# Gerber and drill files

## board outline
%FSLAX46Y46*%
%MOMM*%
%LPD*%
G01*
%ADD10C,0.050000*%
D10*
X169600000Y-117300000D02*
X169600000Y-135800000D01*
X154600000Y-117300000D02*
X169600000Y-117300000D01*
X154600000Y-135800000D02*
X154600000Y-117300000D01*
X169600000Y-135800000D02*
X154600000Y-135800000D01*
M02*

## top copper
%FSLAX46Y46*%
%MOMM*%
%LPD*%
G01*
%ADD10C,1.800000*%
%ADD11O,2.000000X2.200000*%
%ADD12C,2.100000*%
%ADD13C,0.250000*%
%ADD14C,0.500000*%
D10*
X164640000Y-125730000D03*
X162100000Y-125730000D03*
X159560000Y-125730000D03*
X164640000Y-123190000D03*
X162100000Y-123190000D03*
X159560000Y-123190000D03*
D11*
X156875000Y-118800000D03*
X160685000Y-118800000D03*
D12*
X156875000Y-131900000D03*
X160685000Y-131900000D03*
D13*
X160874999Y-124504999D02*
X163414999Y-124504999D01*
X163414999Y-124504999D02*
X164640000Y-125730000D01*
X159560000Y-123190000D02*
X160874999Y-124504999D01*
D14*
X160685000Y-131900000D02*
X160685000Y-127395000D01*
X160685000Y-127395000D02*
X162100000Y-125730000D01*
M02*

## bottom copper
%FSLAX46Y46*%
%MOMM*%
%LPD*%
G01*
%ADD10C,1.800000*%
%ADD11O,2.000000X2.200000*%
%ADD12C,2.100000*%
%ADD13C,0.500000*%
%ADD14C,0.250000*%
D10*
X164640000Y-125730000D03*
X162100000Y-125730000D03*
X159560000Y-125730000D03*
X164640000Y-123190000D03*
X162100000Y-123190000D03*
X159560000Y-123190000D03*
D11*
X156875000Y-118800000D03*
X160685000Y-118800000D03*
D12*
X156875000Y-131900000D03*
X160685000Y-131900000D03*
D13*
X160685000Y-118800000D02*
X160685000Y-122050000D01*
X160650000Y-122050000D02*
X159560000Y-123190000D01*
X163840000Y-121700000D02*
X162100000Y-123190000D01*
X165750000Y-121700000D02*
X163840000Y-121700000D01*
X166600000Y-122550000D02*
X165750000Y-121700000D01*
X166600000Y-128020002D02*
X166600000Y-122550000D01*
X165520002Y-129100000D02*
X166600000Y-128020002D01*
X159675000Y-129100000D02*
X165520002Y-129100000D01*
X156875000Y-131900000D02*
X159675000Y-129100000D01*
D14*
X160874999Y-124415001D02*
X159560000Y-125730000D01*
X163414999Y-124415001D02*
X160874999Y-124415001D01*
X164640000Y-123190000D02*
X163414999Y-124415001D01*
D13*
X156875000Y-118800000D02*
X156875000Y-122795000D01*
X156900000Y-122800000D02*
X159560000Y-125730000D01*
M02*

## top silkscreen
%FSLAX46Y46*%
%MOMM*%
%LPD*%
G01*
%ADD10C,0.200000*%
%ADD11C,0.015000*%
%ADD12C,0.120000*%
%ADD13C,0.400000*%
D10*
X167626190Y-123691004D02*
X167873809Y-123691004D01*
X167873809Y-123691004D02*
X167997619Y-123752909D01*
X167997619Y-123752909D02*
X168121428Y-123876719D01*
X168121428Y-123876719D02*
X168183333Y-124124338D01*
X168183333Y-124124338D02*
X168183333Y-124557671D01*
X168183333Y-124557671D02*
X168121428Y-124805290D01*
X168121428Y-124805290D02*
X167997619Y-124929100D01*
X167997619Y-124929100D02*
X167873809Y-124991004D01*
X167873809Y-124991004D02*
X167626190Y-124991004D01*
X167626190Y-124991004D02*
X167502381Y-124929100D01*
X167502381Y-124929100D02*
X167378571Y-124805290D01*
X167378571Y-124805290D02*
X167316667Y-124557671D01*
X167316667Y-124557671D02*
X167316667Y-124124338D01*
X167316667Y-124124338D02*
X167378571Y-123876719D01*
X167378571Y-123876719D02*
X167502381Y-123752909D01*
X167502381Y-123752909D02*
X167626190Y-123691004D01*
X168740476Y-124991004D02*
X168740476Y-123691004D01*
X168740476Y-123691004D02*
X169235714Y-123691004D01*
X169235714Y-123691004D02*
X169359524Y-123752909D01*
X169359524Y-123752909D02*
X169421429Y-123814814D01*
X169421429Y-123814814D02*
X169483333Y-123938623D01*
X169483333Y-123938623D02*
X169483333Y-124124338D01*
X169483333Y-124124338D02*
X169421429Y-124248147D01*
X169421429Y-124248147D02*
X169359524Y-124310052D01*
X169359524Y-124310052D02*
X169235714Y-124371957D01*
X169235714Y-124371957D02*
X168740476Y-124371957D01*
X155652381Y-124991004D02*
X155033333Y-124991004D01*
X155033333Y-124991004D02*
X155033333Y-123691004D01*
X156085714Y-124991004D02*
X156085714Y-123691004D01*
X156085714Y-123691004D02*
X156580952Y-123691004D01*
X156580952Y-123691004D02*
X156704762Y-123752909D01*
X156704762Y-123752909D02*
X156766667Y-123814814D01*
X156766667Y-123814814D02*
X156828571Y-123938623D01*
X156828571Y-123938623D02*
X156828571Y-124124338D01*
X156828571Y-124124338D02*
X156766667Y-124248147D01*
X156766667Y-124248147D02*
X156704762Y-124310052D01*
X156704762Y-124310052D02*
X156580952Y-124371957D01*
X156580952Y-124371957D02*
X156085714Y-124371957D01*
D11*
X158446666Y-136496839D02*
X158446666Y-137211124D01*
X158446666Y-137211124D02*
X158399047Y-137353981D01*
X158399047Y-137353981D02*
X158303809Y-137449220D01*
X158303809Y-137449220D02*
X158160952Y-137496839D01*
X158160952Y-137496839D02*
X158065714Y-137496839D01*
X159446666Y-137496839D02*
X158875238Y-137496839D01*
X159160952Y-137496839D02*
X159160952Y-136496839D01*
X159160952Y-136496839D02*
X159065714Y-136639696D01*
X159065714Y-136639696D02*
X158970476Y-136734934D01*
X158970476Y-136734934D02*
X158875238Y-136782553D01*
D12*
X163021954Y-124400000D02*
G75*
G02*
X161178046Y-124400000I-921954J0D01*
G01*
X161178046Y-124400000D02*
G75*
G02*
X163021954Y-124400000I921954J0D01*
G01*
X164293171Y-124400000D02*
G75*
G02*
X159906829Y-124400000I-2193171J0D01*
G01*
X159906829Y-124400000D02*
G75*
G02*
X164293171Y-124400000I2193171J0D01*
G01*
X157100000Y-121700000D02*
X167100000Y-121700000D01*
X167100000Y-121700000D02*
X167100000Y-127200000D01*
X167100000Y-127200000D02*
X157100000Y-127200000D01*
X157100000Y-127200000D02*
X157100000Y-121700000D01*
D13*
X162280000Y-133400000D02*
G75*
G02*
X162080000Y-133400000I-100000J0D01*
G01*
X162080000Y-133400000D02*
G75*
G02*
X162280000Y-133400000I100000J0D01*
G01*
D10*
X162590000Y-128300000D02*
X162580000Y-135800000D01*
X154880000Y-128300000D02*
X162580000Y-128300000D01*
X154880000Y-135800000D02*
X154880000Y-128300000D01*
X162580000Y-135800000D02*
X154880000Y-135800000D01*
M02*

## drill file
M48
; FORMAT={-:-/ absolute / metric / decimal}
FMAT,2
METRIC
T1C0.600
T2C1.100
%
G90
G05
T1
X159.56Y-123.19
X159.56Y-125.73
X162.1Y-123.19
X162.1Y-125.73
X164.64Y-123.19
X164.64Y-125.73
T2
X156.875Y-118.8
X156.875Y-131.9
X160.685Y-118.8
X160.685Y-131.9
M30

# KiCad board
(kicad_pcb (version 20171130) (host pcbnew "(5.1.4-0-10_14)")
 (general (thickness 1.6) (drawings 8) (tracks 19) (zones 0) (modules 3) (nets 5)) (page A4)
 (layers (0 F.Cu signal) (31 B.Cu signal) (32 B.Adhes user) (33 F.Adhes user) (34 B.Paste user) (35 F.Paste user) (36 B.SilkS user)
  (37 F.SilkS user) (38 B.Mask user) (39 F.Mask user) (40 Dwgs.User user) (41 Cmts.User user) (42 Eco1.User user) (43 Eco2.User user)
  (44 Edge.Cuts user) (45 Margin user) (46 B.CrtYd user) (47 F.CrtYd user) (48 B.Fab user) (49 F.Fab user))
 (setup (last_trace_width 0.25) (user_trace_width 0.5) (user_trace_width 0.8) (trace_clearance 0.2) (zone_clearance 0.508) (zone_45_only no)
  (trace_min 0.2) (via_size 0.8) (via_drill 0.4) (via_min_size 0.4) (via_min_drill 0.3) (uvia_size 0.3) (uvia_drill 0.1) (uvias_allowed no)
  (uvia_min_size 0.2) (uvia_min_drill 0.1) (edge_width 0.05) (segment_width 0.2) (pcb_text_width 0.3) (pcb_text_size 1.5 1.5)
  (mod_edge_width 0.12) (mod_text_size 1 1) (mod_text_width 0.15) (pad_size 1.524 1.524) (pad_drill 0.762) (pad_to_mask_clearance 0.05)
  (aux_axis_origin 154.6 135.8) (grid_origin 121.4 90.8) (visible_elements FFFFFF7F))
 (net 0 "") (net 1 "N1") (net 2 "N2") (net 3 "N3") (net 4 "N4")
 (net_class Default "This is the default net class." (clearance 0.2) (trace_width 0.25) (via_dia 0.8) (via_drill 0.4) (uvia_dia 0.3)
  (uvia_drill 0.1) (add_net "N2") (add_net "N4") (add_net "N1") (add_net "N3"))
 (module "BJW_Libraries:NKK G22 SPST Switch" (layer F.Cu) (at 162.1 124.5)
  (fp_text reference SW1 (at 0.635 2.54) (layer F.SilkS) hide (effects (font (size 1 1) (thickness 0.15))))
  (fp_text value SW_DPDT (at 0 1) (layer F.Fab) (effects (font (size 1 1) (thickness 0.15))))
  (fp_circle (center 0 -0.1) (end 0.6 0.6) (layer F.SilkS) (width 0.12))
  (fp_circle (center 0 -0.1) (end 1.6 1.4) (layer F.SilkS) (width 0.12))
  (fp_line (start -5 -2.8) (end 5 -2.8) (layer F.SilkS) (width 0.12))
  (fp_line (start 5 -2.8) (end 5 2.7) (layer F.SilkS) (width 0.12))
  (fp_line (start 5 2.7) (end -5 2.7) (layer F.SilkS) (width 0.12))
  (fp_line (start -5 2.7) (end -5 -2.8) (layer F.SilkS) (width 0.12))
  (pad 6 thru_hole circle (at 2.54 1.23) (size 1.8 1.8) (drill 0.6) (layers *.Cu *.Mask) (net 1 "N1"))
  (pad 5 thru_hole circle (at 0 1.23) (size 1.8 1.8) (drill 0.6) (layers *.Cu *.Mask) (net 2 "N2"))
  (pad 4 thru_hole circle (at -2.54 1.23) (size 1.8 1.8) (drill 0.6) (layers *.Cu *.Mask) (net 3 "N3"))
  (pad 3 thru_hole circle (at 2.54 -1.31) (size 1.8 1.8) (drill 0.6) (layers *.Cu *.Mask) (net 3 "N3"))
  (pad 2 thru_hole circle (at 0 -1.31) (size 1.8 1.8) (drill 0.6) (layers *.Cu *.Mask) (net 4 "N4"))
  (pad 1 thru_hole circle (at -2.54 -1.31) (size 1.8 1.8) (drill 0.6) (layers *.Cu *.Mask) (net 1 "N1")))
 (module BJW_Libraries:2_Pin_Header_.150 (layer F.Cu) (at 158.78 118.8 180)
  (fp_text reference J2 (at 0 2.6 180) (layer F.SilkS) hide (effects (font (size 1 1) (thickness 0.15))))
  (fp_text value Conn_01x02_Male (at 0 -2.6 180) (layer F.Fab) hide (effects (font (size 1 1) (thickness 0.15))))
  (pad 2 thru_hole oval (at 1.905 0 180) (size 2 2.2) (drill 1.1) (layers *.Cu *.Mask) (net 3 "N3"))
  (pad 1 thru_hole oval (at -1.905 0 180) (size 2 2.2) (drill 1.1) (layers *.Cu *.Mask) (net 1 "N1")))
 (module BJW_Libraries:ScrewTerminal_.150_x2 (layer F.Cu) (at 158.78 131.9 180)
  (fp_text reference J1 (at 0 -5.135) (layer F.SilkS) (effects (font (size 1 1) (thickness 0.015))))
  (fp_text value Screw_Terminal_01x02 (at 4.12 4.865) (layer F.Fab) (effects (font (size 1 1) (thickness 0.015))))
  (fp_circle (center -3.4 -1.5) (end -3.3 -1.5) (layer F.SilkS) (width 0.4))
  (fp_line (start -3.81 3.6) (end -3.8 -3.9) (layer F.SilkS) (width 0.2))
  (fp_line (start 3.9 3.6) (end -3.8 3.6) (layer F.SilkS) (width 0.2))
  (fp_line (start 3.9 -3.9) (end 3.9 3.6) (layer F.SilkS) (width 0.2))
  (fp_line (start -3.8 -3.9) (end 3.9 -3.9) (layer F.SilkS) (width 0.2))
  (pad 2 thru_hole circle (at 1.905 0 180) (size 2.1 2.1) (drill 1.1) (layers *.Cu *.Mask) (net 4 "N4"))
  (pad 1 thru_hole circle (at -1.905 0 180) (size 2.1 2.1) (drill 1.1) (layers *.Cu *.Mask) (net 2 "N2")))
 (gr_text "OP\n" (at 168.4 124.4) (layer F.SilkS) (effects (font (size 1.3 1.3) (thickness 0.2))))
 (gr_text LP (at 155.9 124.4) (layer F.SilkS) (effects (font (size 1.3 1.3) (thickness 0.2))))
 (gr_line (start 169.6 117.3) (end 169.6 135.8) (layer Edge.Cuts) (width 0.05))
 (gr_line (start 154.6 117.3) (end 169.6 117.3) (layer Edge.Cuts) (width 0.05))
 (gr_line (start 154.6 135.8) (end 154.6 117.3) (layer Edge.Cuts) (width 0.05))
 (gr_line (start 169.6 135.8) (end 154.6 135.8) (layer Edge.Cuts) (width 0.05))
 (segment (start 160.874999 124.504999) (end 163.414999 124.504999) (width 0.25) (layer F.Cu) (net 1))
 (segment (start 163.414999 124.504999) (end 164.64 125.73) (width 0.25) (layer F.Cu) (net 1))
 (segment (start 159.56 123.19) (end 160.874999 124.504999) (width 0.25) (layer F.Cu) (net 1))
 (segment (start 160.685 118.8) (end 160.685 122.05) (width 0.5) (layer B.Cu) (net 1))
 (segment (start 160.65 122.05) (end 159.56 123.19) (width 0.5) (layer B.Cu) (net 1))
 (segment (start 163.84 121.7) (end 162.1 123.19) (width 0.5) (layer B.Cu) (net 4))
 (segment (start 165.75 121.7) (end 163.84 121.7) (width 0.5) (layer B.Cu) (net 4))
 (segment (start 166.6 122.55) (end 165.75 121.7) (width 0.5) (layer B.Cu) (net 4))
 (segment (start 166.6 128.020002) (end 166.6 122.55) (width 0.5) (layer B.Cu) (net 4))
 (segment (start 165.520002 129.1) (end 166.6 128.020002) (width 0.5) (layer B.Cu) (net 4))
 (segment (start 159.675 129.1) (end 165.520002 129.1) (width 0.5) (layer B.Cu) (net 4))
 (segment (start 156.875 131.9) (end 159.675 129.1) (width 0.5) (layer B.Cu) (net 4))
 (segment (start 160.685 131.9) (end 160.685 127.395) (width 0.5) (layer F.Cu) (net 2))
 (segment (start 160.685 127.395) (end 162.1 125.73) (width 0.5) (layer F.Cu) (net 2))
 (segment (start 160.874999 124.415001) (end 159.56 125.73) (width 0.25) (layer B.Cu) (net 3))
 (segment (start 163.414999 124.415001) (end 160.874999 124.415001) (width 0.25) (layer B.Cu) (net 3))
 (segment (start 164.64 123.19) (end 163.414999 124.415001) (width 0.25) (layer B.Cu) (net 3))
 (segment (start 156.875 118.8) (end 156.875 122.795) (width 0.5) (layer B.Cu) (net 3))
 (segment (start 156.9 122.8) (end 159.56 125.73) (width 0.5) (layer B.Cu) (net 3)))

